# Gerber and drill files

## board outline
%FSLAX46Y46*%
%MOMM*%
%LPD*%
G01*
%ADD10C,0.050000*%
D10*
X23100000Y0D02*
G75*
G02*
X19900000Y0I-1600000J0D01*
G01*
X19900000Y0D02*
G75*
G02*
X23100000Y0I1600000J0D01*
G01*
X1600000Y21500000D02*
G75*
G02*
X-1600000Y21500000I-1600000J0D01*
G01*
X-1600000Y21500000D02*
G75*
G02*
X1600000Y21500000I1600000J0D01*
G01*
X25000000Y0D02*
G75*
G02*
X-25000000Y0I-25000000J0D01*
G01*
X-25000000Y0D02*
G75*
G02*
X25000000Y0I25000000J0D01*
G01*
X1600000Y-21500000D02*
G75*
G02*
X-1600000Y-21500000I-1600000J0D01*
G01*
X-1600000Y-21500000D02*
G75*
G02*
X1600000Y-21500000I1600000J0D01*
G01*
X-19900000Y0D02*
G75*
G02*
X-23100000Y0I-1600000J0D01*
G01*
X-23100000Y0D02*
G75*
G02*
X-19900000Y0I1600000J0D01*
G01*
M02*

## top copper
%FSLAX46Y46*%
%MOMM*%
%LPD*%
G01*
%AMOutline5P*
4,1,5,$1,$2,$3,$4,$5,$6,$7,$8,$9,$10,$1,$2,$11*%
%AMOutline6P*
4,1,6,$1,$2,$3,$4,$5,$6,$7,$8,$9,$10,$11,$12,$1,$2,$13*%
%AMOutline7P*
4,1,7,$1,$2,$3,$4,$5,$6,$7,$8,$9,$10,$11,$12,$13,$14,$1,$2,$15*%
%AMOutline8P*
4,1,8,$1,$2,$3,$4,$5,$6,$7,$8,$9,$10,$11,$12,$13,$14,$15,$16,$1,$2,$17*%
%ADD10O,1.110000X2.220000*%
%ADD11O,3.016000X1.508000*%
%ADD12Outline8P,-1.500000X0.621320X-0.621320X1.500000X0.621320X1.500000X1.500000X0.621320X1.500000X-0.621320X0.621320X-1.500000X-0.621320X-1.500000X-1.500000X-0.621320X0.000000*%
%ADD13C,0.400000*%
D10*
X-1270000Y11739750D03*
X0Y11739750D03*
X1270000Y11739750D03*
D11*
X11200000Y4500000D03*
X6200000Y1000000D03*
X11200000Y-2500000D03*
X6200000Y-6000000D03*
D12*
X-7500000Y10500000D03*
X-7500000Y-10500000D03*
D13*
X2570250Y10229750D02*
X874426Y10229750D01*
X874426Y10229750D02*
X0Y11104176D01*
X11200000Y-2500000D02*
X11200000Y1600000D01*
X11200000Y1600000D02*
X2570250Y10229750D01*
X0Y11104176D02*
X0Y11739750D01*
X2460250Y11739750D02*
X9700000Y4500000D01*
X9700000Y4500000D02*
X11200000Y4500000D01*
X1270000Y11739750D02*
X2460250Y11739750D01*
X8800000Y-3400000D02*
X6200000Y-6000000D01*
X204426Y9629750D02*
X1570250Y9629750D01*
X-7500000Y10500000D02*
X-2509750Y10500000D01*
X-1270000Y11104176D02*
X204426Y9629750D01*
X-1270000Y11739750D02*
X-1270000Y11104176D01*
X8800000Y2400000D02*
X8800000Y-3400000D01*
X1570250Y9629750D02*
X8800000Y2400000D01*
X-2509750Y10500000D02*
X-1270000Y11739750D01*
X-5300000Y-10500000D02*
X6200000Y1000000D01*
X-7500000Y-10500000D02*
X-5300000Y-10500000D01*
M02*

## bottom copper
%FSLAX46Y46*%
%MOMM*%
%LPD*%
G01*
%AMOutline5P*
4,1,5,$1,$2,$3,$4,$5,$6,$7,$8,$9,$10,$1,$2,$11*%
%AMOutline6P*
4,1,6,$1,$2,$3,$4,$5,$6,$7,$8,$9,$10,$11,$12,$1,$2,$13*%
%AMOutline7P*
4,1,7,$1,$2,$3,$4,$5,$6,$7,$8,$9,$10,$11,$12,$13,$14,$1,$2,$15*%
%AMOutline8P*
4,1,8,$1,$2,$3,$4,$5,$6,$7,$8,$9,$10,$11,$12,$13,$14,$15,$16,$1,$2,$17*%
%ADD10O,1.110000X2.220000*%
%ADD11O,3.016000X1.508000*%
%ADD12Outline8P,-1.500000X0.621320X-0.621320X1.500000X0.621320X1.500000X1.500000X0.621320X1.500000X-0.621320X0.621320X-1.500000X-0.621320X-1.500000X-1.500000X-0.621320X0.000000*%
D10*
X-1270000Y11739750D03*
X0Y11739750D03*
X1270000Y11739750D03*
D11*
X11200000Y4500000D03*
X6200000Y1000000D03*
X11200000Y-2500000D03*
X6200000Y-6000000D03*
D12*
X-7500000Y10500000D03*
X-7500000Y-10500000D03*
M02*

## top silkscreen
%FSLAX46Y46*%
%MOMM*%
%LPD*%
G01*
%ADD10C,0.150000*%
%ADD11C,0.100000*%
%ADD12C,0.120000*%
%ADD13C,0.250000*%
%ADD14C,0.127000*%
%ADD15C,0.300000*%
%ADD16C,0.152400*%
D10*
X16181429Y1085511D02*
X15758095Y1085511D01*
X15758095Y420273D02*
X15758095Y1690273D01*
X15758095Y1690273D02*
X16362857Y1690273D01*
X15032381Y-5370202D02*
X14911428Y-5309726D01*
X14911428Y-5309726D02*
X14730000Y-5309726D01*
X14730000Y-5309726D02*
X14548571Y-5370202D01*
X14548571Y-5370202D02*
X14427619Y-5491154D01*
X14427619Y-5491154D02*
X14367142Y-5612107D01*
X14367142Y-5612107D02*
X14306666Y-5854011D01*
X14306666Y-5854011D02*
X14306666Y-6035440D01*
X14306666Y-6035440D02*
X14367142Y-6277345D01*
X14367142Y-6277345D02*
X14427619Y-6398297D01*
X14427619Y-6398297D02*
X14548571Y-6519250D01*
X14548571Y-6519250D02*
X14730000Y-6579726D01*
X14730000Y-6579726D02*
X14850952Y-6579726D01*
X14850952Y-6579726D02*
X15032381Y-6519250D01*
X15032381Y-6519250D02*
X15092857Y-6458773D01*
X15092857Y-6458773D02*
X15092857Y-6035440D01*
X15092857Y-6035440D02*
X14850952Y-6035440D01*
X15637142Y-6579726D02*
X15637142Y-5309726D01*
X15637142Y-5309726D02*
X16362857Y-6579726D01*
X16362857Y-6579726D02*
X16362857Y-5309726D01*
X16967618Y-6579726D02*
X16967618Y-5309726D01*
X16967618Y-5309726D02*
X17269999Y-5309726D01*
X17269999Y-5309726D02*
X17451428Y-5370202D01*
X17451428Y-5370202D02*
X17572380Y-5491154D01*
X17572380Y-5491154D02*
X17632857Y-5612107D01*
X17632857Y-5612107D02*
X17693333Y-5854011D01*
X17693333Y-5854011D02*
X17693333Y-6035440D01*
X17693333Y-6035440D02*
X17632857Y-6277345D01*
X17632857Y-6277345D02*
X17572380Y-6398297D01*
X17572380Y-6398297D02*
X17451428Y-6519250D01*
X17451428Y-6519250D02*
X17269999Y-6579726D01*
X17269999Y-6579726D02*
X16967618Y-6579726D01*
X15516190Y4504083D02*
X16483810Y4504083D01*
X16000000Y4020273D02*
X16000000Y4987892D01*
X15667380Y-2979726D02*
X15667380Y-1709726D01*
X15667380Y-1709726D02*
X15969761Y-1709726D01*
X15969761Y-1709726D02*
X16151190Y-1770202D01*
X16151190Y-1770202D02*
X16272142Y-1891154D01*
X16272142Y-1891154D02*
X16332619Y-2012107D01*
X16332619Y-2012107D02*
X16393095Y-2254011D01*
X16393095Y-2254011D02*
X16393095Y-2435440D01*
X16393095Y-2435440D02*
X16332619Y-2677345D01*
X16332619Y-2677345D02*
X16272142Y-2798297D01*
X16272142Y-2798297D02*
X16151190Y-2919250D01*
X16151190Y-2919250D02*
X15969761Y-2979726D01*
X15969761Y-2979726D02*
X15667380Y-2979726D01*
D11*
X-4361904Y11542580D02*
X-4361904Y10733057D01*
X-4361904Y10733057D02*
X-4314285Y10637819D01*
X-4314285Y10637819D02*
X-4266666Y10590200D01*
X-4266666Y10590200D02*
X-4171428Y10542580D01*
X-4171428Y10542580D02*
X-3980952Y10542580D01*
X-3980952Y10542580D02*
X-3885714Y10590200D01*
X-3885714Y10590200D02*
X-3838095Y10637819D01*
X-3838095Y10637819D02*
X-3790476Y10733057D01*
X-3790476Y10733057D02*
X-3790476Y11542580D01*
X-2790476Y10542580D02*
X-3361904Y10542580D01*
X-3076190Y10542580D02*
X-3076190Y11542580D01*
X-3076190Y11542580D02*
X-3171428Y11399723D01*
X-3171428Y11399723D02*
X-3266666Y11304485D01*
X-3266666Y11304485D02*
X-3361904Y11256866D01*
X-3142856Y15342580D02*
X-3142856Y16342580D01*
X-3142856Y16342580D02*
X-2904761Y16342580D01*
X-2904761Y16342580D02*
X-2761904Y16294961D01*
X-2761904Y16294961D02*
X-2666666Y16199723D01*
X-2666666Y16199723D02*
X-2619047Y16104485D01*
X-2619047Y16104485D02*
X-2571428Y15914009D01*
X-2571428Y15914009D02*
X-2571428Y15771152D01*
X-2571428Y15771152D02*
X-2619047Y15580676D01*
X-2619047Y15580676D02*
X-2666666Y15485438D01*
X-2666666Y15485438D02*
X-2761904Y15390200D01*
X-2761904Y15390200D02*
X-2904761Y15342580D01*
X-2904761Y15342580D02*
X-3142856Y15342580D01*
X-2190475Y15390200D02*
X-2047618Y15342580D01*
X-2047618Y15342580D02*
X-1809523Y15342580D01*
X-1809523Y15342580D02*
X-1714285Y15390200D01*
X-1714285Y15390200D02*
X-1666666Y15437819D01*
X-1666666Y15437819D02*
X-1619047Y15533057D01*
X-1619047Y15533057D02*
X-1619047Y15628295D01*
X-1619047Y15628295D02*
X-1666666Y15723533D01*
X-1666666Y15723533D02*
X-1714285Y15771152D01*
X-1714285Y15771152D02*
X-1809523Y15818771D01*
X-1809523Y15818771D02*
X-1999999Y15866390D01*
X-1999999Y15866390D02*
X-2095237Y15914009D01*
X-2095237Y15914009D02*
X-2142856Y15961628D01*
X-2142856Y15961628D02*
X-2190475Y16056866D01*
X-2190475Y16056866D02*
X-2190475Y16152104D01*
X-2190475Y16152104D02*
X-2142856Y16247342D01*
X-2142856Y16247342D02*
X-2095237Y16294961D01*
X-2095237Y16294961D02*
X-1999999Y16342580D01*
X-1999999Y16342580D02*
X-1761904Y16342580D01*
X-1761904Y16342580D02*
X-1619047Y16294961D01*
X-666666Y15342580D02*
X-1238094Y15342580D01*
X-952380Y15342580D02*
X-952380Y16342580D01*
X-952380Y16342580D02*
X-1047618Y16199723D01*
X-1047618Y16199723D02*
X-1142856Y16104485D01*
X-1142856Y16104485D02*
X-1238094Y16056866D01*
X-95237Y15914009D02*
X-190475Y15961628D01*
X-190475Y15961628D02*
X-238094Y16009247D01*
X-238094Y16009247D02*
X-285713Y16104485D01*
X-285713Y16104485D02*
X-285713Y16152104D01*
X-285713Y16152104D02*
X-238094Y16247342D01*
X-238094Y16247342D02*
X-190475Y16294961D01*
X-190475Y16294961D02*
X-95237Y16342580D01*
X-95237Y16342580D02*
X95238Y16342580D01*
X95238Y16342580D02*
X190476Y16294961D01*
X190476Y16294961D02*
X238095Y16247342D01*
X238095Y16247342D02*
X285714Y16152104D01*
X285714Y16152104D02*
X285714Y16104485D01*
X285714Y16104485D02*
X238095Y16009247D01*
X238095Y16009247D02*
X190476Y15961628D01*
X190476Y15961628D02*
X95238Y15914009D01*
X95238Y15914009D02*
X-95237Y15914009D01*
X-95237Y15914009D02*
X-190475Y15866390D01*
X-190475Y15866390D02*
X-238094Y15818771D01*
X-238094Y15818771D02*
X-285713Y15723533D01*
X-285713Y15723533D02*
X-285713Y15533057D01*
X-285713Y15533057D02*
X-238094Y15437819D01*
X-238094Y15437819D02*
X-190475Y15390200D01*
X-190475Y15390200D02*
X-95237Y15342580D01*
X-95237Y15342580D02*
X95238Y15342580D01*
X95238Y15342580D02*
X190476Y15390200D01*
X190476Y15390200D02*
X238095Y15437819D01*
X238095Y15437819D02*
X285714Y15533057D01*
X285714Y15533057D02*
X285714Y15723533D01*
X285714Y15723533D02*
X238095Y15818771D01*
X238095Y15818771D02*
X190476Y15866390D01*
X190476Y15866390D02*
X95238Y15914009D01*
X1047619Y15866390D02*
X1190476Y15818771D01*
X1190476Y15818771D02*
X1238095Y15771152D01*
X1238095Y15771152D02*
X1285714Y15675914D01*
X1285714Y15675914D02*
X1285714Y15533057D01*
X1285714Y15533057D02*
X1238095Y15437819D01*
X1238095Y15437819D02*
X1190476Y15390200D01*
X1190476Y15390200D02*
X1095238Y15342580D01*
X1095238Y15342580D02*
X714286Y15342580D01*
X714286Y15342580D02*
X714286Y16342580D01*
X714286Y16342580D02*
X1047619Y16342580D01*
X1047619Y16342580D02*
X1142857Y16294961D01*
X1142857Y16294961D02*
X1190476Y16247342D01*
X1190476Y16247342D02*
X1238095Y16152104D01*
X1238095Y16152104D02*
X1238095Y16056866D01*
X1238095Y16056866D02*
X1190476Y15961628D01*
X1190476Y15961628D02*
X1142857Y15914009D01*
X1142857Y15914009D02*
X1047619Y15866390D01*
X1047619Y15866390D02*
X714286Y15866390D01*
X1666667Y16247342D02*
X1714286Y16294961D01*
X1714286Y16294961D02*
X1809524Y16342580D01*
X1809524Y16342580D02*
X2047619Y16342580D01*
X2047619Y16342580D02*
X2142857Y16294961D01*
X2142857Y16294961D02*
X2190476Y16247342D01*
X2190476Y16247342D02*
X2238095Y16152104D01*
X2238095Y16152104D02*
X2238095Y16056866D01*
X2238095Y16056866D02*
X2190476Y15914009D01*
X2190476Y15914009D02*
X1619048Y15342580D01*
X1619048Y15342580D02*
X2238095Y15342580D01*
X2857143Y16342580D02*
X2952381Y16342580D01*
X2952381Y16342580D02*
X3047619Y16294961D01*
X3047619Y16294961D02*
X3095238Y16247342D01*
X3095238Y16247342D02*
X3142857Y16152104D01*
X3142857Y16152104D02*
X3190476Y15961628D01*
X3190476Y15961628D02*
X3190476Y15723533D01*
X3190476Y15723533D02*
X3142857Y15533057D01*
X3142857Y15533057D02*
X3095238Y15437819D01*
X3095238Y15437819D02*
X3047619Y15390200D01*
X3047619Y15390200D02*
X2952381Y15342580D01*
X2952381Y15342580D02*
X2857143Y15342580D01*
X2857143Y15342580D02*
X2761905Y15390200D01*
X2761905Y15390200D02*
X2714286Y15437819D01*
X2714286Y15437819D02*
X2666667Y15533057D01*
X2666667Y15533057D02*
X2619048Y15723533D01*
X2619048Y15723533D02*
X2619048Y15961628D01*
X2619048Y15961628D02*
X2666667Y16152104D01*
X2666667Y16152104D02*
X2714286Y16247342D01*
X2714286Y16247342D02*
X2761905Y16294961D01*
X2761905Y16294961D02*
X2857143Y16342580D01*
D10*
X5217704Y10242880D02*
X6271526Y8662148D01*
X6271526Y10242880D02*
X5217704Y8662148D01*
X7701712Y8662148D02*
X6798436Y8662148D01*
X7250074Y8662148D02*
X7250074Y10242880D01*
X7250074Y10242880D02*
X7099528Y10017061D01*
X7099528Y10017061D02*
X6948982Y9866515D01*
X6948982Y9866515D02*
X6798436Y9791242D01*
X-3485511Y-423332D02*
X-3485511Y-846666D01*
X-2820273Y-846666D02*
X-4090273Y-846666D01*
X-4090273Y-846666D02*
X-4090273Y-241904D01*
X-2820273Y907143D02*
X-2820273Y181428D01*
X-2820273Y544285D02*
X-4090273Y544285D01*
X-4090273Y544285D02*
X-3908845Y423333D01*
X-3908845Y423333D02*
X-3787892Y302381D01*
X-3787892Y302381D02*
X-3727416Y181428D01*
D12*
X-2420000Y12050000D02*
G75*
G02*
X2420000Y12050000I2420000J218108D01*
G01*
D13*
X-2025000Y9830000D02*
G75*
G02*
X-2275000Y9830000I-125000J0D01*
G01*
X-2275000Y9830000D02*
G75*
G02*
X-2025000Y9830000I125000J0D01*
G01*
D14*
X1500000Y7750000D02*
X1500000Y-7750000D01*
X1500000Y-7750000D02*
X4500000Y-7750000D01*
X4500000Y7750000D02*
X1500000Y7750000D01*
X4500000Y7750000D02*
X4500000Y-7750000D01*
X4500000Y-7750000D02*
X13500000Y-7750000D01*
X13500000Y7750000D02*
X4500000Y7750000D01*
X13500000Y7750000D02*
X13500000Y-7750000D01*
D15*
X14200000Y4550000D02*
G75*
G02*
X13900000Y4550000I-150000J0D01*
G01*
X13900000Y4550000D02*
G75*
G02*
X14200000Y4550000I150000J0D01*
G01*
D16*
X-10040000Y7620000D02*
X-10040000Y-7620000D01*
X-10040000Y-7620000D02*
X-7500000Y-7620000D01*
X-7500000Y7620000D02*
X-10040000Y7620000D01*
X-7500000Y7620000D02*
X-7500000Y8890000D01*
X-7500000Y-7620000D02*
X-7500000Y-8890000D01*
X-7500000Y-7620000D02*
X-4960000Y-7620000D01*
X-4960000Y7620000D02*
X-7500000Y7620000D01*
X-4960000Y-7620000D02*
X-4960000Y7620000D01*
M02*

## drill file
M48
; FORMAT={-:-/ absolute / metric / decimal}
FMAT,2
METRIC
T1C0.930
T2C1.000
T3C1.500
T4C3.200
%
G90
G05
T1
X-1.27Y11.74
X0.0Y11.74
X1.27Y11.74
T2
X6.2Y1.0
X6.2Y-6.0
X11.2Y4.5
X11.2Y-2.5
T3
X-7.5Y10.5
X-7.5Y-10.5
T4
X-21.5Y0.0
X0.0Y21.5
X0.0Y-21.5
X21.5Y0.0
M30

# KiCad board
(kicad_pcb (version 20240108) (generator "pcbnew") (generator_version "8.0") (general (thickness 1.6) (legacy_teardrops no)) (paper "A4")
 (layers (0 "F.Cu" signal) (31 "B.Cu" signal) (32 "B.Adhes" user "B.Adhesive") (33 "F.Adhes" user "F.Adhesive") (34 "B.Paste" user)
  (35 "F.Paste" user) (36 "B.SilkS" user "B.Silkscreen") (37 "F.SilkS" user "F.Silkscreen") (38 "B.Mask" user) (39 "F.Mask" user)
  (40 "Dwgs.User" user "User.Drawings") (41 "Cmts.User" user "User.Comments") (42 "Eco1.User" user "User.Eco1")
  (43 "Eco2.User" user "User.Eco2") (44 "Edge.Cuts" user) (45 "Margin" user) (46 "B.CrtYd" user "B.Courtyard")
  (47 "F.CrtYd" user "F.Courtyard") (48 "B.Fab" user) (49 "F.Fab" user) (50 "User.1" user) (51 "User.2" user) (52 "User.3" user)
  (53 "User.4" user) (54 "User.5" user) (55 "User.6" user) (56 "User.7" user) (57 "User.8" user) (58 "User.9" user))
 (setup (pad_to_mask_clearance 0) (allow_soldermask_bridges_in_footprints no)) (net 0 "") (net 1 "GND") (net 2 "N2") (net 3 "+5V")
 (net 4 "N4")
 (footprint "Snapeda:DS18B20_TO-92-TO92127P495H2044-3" (layer "F.Cu") (at 0 -12.5)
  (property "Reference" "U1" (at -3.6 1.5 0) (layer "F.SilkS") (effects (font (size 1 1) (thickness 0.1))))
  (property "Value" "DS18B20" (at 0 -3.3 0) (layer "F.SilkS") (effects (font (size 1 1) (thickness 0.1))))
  (fp_arc (start -2.42 0.45) (mid 0 -2.197917) (end 2.42 0.45) (stroke (width 0.12) (type solid)) (layer "F.SilkS"))
  (fp_circle (center -2.15 2.67) (end -2.025 2.67) (stroke (width 0.25) (type solid)) (fill none) (layer "F.SilkS"))
  (pad "1" thru_hole oval (at -1.27 0.76025) (size 1.11 2.22) (drill 0.93) (layers "*.Cu" "*.Mask") (remove_unused_layers no) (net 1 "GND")
   (solder_mask_margin 0.102))
  (pad "2" thru_hole oval (at 0 0.76025) (size 1.11 2.22) (drill 0.93) (layers "*.Cu" "*.Mask") (remove_unused_layers no) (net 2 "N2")
   (solder_mask_margin 0.102))
  (pad "3" thru_hole oval (at 1.27 0.76025) (size 1.11 2.22) (drill 0.93) (layers "*.Cu" "*.Mask") (remove_unused_layers no) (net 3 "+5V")
   (solder_mask_margin 0.102)))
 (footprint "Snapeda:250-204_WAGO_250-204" (layer "F.Cu") (at 7.5 0)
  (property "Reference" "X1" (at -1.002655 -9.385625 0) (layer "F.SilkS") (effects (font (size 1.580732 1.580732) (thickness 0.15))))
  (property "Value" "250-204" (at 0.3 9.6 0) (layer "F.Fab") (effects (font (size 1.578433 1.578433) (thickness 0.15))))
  (fp_line (start -6 -7.75) (end -6 7.75) (stroke (width 0.127) (type solid)) (layer "F.SilkS"))
  (fp_line (start -6 7.75) (end -3 7.75) (stroke (width 0.127) (type solid)) (layer "F.SilkS"))
  (fp_line (start -3 -7.75) (end -6 -7.75) (stroke (width 0.127) (type solid)) (layer "F.SilkS"))
  (fp_line (start -3 -7.75) (end -3 7.75) (stroke (width 0.127) (type solid)) (layer "F.SilkS"))
  (fp_line (start -3 7.75) (end 6 7.75) (stroke (width 0.127) (type solid)) (layer "F.SilkS"))
  (fp_line (start 6 -7.75) (end -3 -7.75) (stroke (width 0.127) (type solid)) (layer "F.SilkS"))
  (fp_line (start 6 -7.75) (end 6 7.75) (stroke (width 0.127) (type solid)) (layer "F.SilkS"))
  (fp_circle (center 6.55 -4.55) (end 6.7 -4.55) (stroke (width 0.3) (type solid)) (fill none) (layer "F.SilkS"))
  (pad "P1" thru_hole oval (at 3.7 -4.5) (size 3.016 1.508) (drill 1) (layers "*.Cu" "*.Mask") (remove_unused_layers no) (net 3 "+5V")
   (solder_mask_margin 0.102))
  (pad "P2" thru_hole oval (at -1.3 -1) (size 3.016 1.508) (drill 1) (layers "*.Cu" "*.Mask") (remove_unused_layers no) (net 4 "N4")
   (solder_mask_margin 0.102))
  (pad "P3" thru_hole oval (at 3.7 2.5) (size 3.016 1.508) (drill 1) (layers "*.Cu" "*.Mask") (remove_unused_layers no) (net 2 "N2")
   (solder_mask_margin 0.102))
  (pad "P4" thru_hole oval (at -1.3 6) (size 3.016 1.508) (drill 1) (layers "*.Cu" "*.Mask") (remove_unused_layers no) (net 1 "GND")
   (solder_mask_margin 0.102)))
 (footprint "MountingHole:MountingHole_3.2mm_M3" (layer "F.Cu") (at 0 -21.5)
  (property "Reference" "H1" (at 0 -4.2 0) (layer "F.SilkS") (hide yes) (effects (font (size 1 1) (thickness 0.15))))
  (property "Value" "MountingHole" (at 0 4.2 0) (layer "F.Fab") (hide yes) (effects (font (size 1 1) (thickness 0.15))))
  (pad "" np_thru_hole circle (at 0 0) (size 3.2 3.2) (drill 3.2) (layers "*.Cu" "*.Mask")))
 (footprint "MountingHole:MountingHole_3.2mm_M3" (layer "F.Cu") (at -21.5 0)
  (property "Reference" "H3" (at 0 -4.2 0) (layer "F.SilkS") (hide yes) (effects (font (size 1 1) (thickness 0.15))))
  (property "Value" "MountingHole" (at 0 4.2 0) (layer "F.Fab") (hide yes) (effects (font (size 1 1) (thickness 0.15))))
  (pad "" np_thru_hole circle (at 0 0) (size 3.2 3.2) (drill 3.2) (layers "*.Cu" "*.Mask")))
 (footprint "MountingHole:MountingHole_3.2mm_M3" (layer "F.Cu") (at 21.5 0)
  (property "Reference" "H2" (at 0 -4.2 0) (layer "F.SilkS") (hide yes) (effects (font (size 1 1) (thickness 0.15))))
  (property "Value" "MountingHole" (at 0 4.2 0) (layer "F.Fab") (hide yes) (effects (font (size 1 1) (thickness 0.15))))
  (pad "" np_thru_hole circle (at 0 0) (size 3.2 3.2) (drill 3.2) (layers "*.Cu" "*.Mask")))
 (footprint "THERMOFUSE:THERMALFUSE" (layer "F.Cu") (at -7.5 0)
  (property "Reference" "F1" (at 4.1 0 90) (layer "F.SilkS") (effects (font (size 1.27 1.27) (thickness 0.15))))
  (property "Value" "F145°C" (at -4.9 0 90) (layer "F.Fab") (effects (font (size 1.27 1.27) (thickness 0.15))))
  (fp_line (start -2.54 -7.62) (end -2.54 7.62) (stroke (width 0.1524) (type solid)) (layer "F.SilkS"))
  (fp_line (start -2.54 7.62) (end 0 7.62) (stroke (width 0.1524) (type solid)) (layer "F.SilkS"))
  (fp_line (start 0 -7.62) (end -2.54 -7.62) (stroke (width 0.1524) (type solid)) (layer "F.SilkS"))
  (fp_line (start 0 -7.62) (end 0 -8.89) (stroke (width 0.1524) (type solid)) (layer "F.SilkS"))
  (fp_line (start 0 7.62) (end 0 8.89) (stroke (width 0.1524) (type solid)) (layer "F.SilkS"))
  (fp_line (start 0 7.62) (end 2.54 7.62) (stroke (width 0.1524) (type solid)) (layer "F.SilkS"))
  (fp_line (start 2.54 -7.62) (end 0 -7.62) (stroke (width 0.1524) (type solid)) (layer "F.SilkS"))
  (fp_line (start 2.54 7.62) (end 2.54 -7.62) (stroke (width 0.1524) (type solid)) (layer "F.SilkS"))
  (pad "1" thru_hole roundrect (at 0 -10.5) (size 3 3) (drill 1.5) (layers "*.Cu" "*.Mask") (remove_unused_layers no)
   (roundrect_rratio 0.25) (chamfer_ratio 0.2928932188) (chamfer top_left top_right bottom_left bottom_right) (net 1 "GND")
   (solder_mask_margin 0.1016) (thermal_bridge_angle 0))
  (pad "2" thru_hole roundrect (at 0 10.5) (size 3 3) (drill 1.5) (layers "*.Cu" "*.Mask") (remove_unused_layers no) (roundrect_rratio 0.25)
   (chamfer_ratio 0.2928932188) (chamfer top_left top_right bottom_left bottom_right) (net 4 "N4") (solder_mask_margin 0.1016)
   (thermal_bridge_angle 0)))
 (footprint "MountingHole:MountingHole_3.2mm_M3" (layer "F.Cu") (at 0 21.5)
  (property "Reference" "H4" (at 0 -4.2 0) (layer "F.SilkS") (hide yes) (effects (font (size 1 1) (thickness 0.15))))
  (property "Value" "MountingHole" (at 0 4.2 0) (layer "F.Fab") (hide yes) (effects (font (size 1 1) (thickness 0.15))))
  (pad "" np_thru_hole circle (at 0 0) (size 3.2 3.2) (drill 3.2) (layers "*.Cu" "*.Mask")))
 (gr_circle (center 21.5 0) (end 23.1 0) (stroke (width 0.05) (type default)) (fill none) (layer "Edge.Cuts"))
 (gr_circle (center 0 -21.5) (end 1.6 -21.5) (stroke (width 0.05) (type default)) (fill none) (layer "Edge.Cuts"))
 (gr_circle (center 0 0) (end 25 0) (stroke (width 0.05) (type default)) (fill none) (layer "Edge.Cuts"))
 (gr_circle (center 0 21.5) (end 1.6 21.5) (stroke (width 0.05) (type default)) (fill none) (layer "Edge.Cuts"))
 (gr_circle (center -21.5 0) (end -19.9 0) (stroke (width 0.05) (type default)) (fill none) (layer "Edge.Cuts"))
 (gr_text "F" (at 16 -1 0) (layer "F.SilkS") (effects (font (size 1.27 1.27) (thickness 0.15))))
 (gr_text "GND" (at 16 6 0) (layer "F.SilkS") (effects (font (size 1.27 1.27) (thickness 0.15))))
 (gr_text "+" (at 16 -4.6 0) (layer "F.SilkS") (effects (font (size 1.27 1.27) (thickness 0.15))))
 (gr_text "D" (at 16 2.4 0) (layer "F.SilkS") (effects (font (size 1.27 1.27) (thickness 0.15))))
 (segment (start 2.57025 -10.22975) (end 0.874426 -10.22975) (width 0.4) (layer "F.Cu") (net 2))
 (segment (start 0.874426 -10.22975) (end 0 -11.104176) (width 0.4) (layer "F.Cu") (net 2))
 (segment (start 11.2 2.5) (end 11.2 -1.6) (width 0.4) (layer "F.Cu") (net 2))
 (segment (start 11.2 -1.6) (end 2.57025 -10.22975) (width 0.4) (layer "F.Cu") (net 2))
 (segment (start 0 -11.104176) (end 0 -11.73975) (width 0.4) (layer "F.Cu") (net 2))
 (segment (start 2.46025 -11.73975) (end 9.7 -4.5) (width 0.4) (layer "F.Cu") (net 3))
 (segment (start 9.7 -4.5) (end 11.2 -4.5) (width 0.4) (layer "F.Cu") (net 3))
 (segment (start 1.27 -11.73975) (end 2.46025 -11.73975) (width 0.4) (layer "F.Cu") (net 3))
 (segment (start 8.8 3.4) (end 6.2 6) (width 0.4) (layer "F.Cu") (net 1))
 (segment (start 0.204426 -9.62975) (end 1.57025 -9.62975) (width 0.4) (layer "F.Cu") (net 1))
 (segment (start -7.5 -10.5) (end -2.50975 -10.5) (width 0.4) (layer "F.Cu") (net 1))
 (segment (start -1.27 -11.104176) (end 0.204426 -9.62975) (width 0.4) (layer "F.Cu") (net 1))
 (segment (start -1.27 -11.73975) (end -1.27 -11.104176) (width 0.4) (layer "F.Cu") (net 1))
 (segment (start 8.8 -2.4) (end 8.8 3.4) (width 0.4) (layer "F.Cu") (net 1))
 (segment (start 1.57025 -9.62975) (end 8.8 -2.4) (width 0.4) (layer "F.Cu") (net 1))
 (segment (start -2.50975 -10.5) (end -1.27 -11.73975) (width 0.4) (layer "F.Cu") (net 1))
 (segment (start -5.3 10.5) (end 6.2 -1) (width 0.4) (layer "F.Cu") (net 4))
 (segment (start -7.5 10.5) (end -5.3 10.5) (width 0.4) (layer "F.Cu") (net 4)))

